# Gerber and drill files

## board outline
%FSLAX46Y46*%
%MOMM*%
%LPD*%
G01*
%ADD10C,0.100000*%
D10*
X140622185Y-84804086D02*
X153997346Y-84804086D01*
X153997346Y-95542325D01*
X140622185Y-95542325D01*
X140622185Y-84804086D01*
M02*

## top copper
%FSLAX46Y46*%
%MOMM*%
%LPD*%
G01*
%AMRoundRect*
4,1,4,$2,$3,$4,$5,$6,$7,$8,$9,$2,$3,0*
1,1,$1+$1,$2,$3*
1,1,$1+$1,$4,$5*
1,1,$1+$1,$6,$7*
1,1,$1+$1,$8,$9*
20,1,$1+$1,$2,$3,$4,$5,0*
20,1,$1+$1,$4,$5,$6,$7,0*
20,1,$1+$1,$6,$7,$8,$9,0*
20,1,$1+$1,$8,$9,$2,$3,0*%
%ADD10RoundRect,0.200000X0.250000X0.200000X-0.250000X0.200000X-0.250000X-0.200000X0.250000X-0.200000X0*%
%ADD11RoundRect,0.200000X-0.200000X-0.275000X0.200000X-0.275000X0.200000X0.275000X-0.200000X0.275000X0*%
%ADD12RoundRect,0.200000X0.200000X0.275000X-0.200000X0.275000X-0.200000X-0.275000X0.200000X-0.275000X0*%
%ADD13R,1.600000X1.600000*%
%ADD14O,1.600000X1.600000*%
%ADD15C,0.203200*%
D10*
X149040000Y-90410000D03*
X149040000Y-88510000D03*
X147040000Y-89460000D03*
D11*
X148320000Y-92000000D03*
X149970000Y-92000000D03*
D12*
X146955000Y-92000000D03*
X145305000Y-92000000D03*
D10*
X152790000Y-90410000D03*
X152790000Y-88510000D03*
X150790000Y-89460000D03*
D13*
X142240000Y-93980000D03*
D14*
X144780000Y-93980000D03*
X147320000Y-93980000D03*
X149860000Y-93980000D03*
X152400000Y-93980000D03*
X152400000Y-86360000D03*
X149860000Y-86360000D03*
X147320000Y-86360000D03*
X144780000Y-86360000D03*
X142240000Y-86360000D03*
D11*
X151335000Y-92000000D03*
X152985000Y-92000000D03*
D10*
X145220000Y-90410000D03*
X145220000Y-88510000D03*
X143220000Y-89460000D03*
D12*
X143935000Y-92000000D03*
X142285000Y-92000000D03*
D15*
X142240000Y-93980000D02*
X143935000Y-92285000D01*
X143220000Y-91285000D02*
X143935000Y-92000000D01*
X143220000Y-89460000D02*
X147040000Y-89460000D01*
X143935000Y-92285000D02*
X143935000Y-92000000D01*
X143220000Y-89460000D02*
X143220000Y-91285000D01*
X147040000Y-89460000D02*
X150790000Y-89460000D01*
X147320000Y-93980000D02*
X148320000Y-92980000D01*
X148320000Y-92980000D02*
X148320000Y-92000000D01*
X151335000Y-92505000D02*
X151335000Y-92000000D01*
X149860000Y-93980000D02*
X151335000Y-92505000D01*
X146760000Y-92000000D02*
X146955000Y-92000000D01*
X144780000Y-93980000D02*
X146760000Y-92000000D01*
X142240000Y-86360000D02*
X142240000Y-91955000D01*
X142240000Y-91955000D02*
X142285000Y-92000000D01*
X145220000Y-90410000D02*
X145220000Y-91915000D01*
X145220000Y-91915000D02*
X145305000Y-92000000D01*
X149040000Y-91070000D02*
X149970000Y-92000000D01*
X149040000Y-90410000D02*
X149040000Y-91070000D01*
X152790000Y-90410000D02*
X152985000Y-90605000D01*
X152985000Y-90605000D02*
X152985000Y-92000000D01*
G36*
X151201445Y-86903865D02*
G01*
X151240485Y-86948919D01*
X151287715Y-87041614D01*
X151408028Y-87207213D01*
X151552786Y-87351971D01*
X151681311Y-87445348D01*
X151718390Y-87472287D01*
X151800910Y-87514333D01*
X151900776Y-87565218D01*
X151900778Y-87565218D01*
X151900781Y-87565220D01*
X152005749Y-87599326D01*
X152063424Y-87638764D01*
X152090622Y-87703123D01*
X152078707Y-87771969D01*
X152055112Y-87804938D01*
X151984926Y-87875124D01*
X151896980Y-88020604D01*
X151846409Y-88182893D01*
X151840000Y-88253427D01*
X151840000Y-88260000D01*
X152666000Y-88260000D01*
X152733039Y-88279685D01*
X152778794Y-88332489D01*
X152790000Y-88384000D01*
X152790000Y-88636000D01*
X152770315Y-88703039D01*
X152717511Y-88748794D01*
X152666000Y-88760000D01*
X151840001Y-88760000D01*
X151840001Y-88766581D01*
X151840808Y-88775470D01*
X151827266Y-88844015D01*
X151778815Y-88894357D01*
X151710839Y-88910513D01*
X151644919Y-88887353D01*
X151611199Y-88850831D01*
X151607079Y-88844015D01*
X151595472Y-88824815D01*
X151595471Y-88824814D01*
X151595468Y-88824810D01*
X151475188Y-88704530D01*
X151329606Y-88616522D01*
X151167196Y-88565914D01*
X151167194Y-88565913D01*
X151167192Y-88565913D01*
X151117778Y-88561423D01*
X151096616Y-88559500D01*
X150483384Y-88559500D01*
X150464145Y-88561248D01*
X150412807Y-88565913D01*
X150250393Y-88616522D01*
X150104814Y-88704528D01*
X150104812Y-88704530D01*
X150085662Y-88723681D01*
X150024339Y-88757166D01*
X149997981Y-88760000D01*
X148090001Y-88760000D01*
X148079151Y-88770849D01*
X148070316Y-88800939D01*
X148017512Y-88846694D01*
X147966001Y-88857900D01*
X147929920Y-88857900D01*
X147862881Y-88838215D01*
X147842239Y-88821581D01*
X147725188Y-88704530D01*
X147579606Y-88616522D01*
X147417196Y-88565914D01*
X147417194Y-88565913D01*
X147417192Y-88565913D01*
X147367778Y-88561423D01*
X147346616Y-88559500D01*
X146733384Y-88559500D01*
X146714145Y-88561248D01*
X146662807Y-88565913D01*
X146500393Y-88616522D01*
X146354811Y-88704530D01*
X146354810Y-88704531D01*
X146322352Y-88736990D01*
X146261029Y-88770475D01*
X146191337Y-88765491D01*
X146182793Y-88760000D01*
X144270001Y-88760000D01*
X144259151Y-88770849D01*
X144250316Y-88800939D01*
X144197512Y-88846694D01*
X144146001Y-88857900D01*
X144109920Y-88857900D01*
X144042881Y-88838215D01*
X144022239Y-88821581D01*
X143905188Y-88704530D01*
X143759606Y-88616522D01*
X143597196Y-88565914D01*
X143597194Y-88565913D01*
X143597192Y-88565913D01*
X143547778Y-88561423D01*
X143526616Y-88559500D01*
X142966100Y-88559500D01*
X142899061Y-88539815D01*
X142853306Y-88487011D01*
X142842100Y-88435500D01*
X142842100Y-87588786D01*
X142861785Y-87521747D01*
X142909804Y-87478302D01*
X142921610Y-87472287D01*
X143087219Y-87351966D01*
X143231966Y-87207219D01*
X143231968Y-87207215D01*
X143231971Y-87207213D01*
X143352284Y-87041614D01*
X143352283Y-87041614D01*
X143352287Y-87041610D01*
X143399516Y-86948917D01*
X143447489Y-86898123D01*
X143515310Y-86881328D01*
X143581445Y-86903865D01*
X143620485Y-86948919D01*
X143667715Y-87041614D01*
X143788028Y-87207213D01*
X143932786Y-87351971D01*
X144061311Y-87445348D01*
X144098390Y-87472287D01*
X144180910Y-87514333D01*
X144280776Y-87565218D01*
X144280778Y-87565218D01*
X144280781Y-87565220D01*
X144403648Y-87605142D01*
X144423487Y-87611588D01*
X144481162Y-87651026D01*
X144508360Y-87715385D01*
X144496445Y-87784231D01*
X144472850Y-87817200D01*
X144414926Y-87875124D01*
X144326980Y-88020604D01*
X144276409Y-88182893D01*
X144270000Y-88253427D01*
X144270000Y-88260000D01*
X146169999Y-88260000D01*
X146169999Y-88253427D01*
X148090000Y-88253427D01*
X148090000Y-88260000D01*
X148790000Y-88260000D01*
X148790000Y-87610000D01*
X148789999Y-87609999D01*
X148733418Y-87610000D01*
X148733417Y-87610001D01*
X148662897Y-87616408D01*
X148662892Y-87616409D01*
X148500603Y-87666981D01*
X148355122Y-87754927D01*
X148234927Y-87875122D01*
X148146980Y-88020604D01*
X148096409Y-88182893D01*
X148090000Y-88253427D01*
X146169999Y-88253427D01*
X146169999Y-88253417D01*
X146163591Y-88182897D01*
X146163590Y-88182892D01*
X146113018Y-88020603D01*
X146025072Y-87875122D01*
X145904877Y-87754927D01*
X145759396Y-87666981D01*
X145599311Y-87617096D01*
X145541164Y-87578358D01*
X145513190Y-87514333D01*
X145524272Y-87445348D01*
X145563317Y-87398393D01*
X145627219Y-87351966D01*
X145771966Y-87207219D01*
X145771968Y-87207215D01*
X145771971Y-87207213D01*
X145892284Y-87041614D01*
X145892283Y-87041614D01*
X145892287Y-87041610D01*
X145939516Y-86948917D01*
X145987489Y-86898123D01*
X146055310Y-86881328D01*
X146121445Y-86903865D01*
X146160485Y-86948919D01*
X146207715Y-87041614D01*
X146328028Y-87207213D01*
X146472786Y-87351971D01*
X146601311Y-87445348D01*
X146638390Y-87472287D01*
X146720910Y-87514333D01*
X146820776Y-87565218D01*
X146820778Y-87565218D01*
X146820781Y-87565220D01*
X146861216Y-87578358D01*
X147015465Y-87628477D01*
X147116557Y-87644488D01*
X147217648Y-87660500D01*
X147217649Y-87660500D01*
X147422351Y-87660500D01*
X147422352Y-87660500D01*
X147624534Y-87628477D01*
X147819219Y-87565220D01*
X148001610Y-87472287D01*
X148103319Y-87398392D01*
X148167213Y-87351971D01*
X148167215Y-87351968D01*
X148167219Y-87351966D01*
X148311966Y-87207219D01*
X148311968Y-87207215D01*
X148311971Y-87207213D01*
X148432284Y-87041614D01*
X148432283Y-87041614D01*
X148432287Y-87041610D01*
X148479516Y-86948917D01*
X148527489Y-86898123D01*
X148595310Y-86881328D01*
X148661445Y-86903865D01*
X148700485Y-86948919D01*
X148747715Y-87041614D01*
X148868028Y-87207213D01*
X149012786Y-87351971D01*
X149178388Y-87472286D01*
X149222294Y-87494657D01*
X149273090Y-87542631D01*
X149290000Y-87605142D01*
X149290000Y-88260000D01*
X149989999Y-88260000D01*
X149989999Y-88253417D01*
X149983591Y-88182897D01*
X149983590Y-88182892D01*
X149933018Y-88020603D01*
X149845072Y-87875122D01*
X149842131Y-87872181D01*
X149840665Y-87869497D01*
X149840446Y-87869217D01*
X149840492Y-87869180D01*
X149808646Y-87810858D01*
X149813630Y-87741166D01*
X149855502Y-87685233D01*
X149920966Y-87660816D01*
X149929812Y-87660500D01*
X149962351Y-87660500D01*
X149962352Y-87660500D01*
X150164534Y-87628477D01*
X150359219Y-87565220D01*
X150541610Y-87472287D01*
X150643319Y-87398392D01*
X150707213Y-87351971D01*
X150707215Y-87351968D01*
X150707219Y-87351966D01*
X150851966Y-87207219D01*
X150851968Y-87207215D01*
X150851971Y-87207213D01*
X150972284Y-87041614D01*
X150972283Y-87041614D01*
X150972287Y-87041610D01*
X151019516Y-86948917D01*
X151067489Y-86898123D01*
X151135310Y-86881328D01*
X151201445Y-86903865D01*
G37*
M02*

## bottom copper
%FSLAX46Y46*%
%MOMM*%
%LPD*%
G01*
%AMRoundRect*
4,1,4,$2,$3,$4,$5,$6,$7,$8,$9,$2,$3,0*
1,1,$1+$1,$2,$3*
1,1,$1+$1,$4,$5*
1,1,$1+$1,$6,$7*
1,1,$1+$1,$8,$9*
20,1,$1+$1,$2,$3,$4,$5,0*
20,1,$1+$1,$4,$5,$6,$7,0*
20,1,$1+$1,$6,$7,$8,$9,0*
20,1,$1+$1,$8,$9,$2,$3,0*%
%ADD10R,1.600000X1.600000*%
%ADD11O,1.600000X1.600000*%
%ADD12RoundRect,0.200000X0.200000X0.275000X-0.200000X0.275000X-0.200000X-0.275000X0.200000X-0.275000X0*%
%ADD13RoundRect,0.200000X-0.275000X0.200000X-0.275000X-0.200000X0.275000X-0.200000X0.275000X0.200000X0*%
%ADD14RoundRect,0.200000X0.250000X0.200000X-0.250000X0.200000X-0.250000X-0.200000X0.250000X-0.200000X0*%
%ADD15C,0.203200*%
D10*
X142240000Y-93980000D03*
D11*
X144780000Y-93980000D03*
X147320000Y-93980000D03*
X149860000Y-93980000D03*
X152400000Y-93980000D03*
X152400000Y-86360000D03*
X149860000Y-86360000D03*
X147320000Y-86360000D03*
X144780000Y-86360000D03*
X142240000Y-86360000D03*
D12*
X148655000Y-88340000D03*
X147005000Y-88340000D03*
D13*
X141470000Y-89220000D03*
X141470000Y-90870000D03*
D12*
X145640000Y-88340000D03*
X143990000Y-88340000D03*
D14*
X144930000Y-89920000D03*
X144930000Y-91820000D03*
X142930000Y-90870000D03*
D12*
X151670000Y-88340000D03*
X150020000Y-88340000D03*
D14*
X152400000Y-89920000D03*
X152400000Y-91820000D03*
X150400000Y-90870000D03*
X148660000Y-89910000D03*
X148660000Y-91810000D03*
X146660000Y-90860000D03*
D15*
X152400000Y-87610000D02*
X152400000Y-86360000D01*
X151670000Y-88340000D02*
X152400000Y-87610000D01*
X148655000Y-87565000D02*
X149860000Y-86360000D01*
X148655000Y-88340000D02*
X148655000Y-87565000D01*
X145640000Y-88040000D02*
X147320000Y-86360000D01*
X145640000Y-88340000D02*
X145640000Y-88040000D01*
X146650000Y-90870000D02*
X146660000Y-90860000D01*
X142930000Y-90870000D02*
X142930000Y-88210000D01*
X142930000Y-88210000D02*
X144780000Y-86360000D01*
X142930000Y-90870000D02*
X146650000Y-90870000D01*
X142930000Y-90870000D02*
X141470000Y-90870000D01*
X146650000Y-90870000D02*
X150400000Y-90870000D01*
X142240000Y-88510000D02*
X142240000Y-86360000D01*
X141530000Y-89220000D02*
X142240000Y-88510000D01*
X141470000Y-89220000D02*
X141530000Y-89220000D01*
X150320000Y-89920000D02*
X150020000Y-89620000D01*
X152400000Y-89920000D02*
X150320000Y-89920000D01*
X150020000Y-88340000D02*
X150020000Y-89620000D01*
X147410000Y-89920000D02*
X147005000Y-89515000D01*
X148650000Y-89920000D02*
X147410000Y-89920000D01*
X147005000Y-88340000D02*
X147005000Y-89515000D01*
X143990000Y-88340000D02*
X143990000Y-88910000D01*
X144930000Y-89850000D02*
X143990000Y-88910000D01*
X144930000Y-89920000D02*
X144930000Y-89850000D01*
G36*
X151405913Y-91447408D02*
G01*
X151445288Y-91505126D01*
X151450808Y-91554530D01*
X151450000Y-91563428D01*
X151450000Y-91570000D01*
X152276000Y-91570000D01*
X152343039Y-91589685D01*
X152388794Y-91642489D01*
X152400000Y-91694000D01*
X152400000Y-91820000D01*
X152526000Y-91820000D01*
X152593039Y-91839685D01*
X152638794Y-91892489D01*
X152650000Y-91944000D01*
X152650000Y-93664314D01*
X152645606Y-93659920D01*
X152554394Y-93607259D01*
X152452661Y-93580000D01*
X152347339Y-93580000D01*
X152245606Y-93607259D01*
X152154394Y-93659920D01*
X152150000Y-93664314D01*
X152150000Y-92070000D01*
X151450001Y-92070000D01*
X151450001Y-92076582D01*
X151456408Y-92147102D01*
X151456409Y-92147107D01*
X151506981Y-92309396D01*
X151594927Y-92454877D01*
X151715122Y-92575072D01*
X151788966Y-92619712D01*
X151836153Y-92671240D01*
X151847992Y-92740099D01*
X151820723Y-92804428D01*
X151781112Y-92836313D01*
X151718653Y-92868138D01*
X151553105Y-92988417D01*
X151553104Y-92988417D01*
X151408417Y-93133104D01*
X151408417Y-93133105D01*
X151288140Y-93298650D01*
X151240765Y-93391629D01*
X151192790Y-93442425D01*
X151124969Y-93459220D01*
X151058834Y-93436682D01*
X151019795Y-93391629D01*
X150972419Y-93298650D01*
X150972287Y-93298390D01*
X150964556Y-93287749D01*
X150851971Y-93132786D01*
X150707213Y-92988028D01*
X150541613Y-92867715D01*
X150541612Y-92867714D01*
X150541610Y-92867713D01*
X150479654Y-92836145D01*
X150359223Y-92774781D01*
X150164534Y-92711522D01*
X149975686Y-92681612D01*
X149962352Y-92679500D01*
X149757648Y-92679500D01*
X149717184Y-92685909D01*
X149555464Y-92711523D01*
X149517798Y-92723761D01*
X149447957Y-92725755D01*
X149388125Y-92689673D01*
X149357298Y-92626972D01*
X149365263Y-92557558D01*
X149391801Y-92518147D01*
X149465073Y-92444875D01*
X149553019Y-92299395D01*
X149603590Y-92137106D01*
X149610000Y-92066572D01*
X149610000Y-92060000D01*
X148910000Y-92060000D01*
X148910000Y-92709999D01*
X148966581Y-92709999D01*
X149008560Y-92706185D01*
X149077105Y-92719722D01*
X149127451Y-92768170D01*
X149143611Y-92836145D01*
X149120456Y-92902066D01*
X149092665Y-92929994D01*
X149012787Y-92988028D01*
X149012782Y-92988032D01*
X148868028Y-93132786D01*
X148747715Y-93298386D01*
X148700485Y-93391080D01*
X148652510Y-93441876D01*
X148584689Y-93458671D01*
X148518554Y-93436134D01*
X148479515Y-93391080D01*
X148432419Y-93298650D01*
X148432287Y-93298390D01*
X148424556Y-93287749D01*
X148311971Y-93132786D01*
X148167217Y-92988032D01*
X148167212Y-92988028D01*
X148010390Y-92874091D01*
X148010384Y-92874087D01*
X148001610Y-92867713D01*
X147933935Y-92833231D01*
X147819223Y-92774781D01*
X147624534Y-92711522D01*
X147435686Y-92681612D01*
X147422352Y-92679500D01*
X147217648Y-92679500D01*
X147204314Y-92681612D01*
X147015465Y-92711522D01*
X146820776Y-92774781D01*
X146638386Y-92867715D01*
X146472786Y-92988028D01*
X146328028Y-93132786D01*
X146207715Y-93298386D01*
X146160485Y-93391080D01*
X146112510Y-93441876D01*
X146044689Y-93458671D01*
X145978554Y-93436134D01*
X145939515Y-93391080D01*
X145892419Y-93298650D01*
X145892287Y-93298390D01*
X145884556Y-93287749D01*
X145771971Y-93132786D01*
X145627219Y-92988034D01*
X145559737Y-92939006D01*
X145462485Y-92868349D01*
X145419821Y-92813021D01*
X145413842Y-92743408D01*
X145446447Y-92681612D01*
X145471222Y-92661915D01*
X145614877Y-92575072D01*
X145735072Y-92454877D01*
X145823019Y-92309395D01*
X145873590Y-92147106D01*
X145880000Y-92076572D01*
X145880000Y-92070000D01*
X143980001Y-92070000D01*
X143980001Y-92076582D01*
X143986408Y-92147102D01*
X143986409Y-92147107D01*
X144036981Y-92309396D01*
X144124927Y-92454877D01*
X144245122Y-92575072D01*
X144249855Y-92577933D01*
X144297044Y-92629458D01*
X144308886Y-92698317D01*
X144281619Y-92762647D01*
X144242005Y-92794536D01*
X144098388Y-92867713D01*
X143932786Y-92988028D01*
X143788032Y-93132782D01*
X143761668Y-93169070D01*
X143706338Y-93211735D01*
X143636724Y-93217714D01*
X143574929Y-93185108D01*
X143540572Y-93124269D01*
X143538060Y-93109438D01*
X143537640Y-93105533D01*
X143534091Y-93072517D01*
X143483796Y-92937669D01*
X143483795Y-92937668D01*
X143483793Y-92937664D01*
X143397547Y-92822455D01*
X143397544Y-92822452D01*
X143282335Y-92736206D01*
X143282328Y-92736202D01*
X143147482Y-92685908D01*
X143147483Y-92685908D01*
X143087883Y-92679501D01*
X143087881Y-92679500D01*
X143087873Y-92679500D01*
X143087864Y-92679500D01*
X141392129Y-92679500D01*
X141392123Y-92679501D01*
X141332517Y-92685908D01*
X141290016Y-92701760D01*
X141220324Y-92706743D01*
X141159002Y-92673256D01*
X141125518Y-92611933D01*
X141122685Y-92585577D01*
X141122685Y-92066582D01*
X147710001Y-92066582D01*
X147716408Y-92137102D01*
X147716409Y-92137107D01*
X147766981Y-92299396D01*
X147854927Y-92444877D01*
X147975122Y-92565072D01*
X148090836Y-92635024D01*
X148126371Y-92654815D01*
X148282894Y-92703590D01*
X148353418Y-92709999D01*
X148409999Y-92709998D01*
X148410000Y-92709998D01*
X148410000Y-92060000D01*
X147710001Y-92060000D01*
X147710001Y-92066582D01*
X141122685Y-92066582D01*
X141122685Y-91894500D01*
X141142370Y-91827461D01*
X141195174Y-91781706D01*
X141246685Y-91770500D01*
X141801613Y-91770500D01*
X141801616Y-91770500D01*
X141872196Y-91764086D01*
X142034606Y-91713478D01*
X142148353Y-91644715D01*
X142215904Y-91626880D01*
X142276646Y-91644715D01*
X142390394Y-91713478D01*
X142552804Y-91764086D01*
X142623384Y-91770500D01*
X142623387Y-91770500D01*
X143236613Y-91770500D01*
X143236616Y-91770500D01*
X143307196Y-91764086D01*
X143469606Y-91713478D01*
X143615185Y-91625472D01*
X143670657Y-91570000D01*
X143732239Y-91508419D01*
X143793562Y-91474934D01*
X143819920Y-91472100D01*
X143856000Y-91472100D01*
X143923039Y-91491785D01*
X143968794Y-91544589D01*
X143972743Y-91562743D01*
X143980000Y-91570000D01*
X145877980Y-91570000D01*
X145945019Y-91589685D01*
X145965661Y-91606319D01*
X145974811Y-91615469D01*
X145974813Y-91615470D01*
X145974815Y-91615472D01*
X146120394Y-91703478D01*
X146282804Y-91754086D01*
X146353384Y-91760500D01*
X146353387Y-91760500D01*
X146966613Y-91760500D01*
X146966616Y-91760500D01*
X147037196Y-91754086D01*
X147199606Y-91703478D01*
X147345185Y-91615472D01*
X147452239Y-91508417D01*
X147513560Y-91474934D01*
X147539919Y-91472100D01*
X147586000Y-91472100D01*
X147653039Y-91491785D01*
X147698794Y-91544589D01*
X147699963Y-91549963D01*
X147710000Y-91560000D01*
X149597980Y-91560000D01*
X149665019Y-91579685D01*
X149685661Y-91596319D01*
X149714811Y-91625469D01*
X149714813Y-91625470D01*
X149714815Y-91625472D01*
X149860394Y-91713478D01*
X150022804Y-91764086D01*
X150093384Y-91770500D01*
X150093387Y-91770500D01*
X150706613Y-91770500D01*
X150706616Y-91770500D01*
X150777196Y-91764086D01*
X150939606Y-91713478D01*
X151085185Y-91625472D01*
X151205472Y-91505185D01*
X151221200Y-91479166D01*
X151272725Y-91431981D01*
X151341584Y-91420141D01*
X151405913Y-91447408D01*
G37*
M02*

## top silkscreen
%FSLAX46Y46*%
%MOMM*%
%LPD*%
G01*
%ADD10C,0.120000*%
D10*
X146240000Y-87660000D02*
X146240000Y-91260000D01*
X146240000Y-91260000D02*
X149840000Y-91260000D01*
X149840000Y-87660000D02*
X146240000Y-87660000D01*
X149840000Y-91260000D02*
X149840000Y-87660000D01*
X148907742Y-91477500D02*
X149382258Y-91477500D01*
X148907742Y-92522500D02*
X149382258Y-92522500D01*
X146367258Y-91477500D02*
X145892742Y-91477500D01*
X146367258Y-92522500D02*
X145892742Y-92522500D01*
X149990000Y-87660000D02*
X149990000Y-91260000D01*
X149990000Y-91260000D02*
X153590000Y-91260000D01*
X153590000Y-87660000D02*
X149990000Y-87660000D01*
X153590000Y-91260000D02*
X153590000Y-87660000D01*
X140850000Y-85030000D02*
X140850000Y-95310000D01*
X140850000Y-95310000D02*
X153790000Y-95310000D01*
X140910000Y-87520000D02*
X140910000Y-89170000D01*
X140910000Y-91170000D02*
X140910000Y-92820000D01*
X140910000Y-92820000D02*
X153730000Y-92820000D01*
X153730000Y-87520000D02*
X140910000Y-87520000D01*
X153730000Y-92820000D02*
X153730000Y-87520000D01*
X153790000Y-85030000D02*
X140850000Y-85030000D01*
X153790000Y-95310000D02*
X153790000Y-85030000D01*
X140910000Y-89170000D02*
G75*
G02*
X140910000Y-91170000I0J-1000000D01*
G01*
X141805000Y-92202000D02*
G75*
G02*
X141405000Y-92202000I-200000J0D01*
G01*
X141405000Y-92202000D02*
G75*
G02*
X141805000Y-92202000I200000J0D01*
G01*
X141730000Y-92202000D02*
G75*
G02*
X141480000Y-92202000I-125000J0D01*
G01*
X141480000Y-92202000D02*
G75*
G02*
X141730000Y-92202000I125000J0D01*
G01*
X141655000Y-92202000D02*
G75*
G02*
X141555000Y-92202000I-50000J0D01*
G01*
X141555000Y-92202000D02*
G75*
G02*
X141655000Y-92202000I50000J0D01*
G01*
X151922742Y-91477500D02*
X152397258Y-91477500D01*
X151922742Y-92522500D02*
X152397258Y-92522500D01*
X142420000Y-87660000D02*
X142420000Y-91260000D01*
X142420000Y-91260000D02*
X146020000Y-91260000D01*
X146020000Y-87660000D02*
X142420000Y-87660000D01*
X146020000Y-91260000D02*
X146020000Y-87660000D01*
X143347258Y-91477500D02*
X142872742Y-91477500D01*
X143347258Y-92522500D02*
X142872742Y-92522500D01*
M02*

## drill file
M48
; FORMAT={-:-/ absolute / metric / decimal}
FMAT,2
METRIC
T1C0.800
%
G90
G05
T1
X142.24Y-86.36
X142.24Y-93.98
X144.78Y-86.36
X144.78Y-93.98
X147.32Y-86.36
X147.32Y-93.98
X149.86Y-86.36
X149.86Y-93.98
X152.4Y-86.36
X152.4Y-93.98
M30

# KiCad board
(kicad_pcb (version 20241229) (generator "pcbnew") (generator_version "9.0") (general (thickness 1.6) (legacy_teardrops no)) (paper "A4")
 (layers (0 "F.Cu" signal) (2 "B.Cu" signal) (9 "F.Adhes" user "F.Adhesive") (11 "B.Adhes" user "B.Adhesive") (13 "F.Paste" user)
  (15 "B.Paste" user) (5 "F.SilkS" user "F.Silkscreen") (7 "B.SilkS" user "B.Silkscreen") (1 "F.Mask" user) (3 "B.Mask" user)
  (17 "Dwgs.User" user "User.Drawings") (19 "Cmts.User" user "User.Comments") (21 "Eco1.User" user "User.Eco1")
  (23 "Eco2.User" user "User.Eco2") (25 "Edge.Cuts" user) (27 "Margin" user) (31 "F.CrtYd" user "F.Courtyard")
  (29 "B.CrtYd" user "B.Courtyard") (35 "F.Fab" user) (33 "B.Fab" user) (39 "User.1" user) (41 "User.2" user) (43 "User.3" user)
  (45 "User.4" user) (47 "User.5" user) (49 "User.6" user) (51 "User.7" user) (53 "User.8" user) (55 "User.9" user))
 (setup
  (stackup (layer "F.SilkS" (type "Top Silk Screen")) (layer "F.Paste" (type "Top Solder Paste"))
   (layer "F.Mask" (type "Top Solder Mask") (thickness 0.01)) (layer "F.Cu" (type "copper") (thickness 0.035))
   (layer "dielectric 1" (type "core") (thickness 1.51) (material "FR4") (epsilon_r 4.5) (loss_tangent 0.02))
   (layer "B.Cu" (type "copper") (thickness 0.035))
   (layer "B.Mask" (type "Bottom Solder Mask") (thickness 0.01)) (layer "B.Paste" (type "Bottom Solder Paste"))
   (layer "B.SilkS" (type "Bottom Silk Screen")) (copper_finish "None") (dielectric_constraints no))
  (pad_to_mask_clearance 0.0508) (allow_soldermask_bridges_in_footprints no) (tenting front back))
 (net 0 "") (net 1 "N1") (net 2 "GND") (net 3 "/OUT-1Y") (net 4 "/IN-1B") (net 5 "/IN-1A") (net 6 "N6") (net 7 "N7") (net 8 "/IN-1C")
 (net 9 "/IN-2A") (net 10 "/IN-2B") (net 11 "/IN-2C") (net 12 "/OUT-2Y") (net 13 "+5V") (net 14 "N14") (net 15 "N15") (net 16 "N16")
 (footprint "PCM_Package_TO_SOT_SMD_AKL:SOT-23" (layer "F.Cu") (at 148.04 89.46 180)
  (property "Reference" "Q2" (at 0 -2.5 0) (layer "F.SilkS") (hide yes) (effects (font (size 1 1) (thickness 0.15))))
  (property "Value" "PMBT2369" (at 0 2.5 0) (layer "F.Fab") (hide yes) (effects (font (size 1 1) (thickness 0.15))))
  (fp_line (start 1.8 1.8) (end 1.8 -1.8) (stroke (width 0.12) (type solid)) (layer "F.SilkS"))
  (fp_line (start 1.8 -1.8) (end -1.8 -1.8) (stroke (width 0.12) (type solid)) (layer "F.SilkS"))
  (fp_line (start -1.8 1.8) (end 1.8 1.8) (stroke (width 0.12) (type solid)) (layer "F.SilkS"))
  (fp_line (start -1.8 -1.8) (end -1.8 1.8) (stroke (width 0.12) (type solid)) (layer "F.SilkS"))
  (pad "1" smd roundrect (at -1 -0.95 180) (size 0.9 0.8) (layers "F.Cu" "F.Mask" "F.Paste") (roundrect_rratio 0.25) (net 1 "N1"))
  (pad "2" smd roundrect (at -1 0.95 180) (size 0.9 0.8) (layers "F.Cu" "F.Mask" "F.Paste") (roundrect_rratio 0.25) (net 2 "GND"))
  (pad "3" smd roundrect (at 1 0 180) (size 0.9 0.8) (layers "F.Cu" "F.Mask" "F.Paste") (roundrect_rratio 0.25) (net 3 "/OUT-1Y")))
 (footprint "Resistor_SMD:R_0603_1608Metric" (layer "F.Cu") (at 149.145 92)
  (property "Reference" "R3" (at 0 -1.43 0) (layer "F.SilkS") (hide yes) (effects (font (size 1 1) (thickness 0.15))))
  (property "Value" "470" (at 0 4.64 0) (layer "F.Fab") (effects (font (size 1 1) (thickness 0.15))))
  (fp_line (start -0.237258 -0.5225) (end 0.237258 -0.5225) (stroke (width 0.12) (type solid)) (layer "F.SilkS"))
  (fp_line (start -0.237258 0.5225) (end 0.237258 0.5225) (stroke (width 0.12) (type solid)) (layer "F.SilkS"))
  (pad "1" smd roundrect (at -0.825 0) (size 0.8 0.95) (layers "F.Cu" "F.Mask" "F.Paste") (roundrect_rratio 0.25) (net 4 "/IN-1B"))
  (pad "2" smd roundrect (at 0.825 0) (size 0.8 0.95) (layers "F.Cu" "F.Mask" "F.Paste") (roundrect_rratio 0.25) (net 1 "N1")))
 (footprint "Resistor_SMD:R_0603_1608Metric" (layer "F.Cu") (at 146.13 92 180)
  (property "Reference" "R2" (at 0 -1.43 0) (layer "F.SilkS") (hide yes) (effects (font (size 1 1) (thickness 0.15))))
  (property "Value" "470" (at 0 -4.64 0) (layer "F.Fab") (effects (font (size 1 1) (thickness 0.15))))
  (fp_line (start -0.237258 0.5225) (end 0.237258 0.5225) (stroke (width 0.12) (type solid)) (layer "F.SilkS"))
  (fp_line (start -0.237258 -0.5225) (end 0.237258 -0.5225) (stroke (width 0.12) (type solid)) (layer "F.SilkS"))
  (pad "1" smd roundrect (at -0.825 0 180) (size 0.8 0.95) (layers "F.Cu" "F.Mask" "F.Paste") (roundrect_rratio 0.25) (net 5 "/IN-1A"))
  (pad "2" smd roundrect (at 0.825 0 180) (size 0.8 0.95) (layers "F.Cu" "F.Mask" "F.Paste") (roundrect_rratio 0.25) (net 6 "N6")))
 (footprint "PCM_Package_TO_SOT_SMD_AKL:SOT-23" (layer "F.Cu") (at 151.79 89.46 180)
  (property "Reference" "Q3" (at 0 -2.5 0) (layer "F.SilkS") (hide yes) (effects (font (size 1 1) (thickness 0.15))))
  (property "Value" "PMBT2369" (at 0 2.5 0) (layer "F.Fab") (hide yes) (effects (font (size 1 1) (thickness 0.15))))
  (fp_line (start 1.8 1.8) (end 1.8 -1.8) (stroke (width 0.12) (type solid)) (layer "F.SilkS"))
  (fp_line (start 1.8 -1.8) (end -1.8 -1.8) (stroke (width 0.12) (type solid)) (layer "F.SilkS"))
  (fp_line (start -1.8 1.8) (end 1.8 1.8) (stroke (width 0.12) (type solid)) (layer "F.SilkS"))
  (fp_line (start -1.8 -1.8) (end -1.8 1.8) (stroke (width 0.12) (type solid)) (layer "F.SilkS"))
  (pad "1" smd roundrect (at -1 -0.95 180) (size 0.9 0.8) (layers "F.Cu" "F.Mask" "F.Paste") (roundrect_rratio 0.25) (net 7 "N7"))
  (pad "2" smd roundrect (at -1 0.95 180) (size 0.9 0.8) (layers "F.Cu" "F.Mask" "F.Paste") (roundrect_rratio 0.25) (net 2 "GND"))
  (pad "3" smd roundrect (at 1 0 180) (size 0.9 0.8) (layers "F.Cu" "F.Mask" "F.Paste") (roundrect_rratio 0.25) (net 3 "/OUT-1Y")))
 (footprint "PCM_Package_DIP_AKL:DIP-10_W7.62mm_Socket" (layer "F.Cu") (at 142.24 93.98 90)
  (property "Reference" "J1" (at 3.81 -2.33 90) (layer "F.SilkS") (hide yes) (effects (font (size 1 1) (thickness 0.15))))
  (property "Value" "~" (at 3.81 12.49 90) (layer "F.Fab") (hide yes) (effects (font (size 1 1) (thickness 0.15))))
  (fp_line (start 8.95 -1.39) (end -1.33 -1.39) (stroke (width 0.12) (type solid)) (layer "F.SilkS"))
  (fp_line (start -1.33 -1.39) (end -1.33 11.55) (stroke (width 0.12) (type solid)) (layer "F.SilkS"))
  (fp_line (start 6.46 -1.33) (end 4.81 -1.33) (stroke (width 0.12) (type solid)) (layer "F.SilkS"))
  (fp_line (start 2.81 -1.33) (end 1.16 -1.33) (stroke (width 0.12) (type solid)) (layer "F.SilkS"))
  (fp_line (start 1.16 -1.33) (end 1.16 11.49) (stroke (width 0.12) (type solid)) (layer "F.SilkS"))
  (fp_line (start 6.46 11.49) (end 6.46 -1.33) (stroke (width 0.12) (type solid)) (layer "F.SilkS"))
  (fp_line (start 1.16 11.49) (end 6.46 11.49) (stroke (width 0.12) (type solid)) (layer "F.SilkS"))
  (fp_line (start 8.95 11.55) (end 8.95 -1.39) (stroke (width 0.12) (type solid)) (layer "F.SilkS"))
  (fp_line (start -1.33 11.55) (end 8.95 11.55) (stroke (width 0.12) (type solid)) (layer "F.SilkS"))
  (fp_arc (start 4.81 -1.33) (mid 3.81 -0.33) (end 2.81 -1.33) (stroke (width 0.12) (type solid)) (layer "F.SilkS"))
  (fp_circle (center 1.778 -0.635) (end 1.978 -0.635) (stroke (width 0.12) (type solid)) (fill no) (layer "F.SilkS"))
  (fp_circle (center 1.778 -0.635) (end 1.903 -0.635) (stroke (width 0.12) (type solid)) (fill no) (layer "F.SilkS"))
  (fp_circle (center 1.778 -0.635) (end 1.828 -0.635) (stroke (width 0.12) (type solid)) (fill no) (layer "F.SilkS"))
  (pad "1" thru_hole rect (at 0 0 90) (size 1.6 1.6) (drill 0.8) (layers "*.Cu" "*.Mask") (remove_unused_layers no) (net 3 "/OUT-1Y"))
  (pad "2" thru_hole oval (at 0 2.54 90) (size 1.6 1.6) (drill 0.8) (layers "*.Cu" "*.Mask") (remove_unused_layers no) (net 5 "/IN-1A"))
  (pad "3" thru_hole oval (at 0 5.08 90) (size 1.6 1.6) (drill 0.8) (layers "*.Cu" "*.Mask") (remove_unused_layers no) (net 4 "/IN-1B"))
  (pad "4" thru_hole oval (at 0 7.62 90) (size 1.6 1.6) (drill 0.8) (layers "*.Cu" "*.Mask") (remove_unused_layers no) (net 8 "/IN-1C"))
  (pad "5" thru_hole oval (at 0 10.16 90) (size 1.6 1.6) (drill 0.8) (layers "*.Cu" "*.Mask") (remove_unused_layers no) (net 2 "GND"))
  (pad "6" thru_hole oval (at 7.62 10.16 90) (size 1.6 1.6) (drill 0.8) (layers "*.Cu" "*.Mask") (remove_unused_layers no) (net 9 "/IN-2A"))
  (pad "7" thru_hole oval (at 7.62 7.62 90) (size 1.6 1.6) (drill 0.8) (layers "*.Cu" "*.Mask") (remove_unused_layers no) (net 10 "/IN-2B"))
  (pad "8" thru_hole oval (at 7.62 5.08 90) (size 1.6 1.6) (drill 0.8) (layers "*.Cu" "*.Mask") (remove_unused_layers no) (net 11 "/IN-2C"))
  (pad "9" thru_hole oval (at 7.62 2.54 90) (size 1.6 1.6) (drill 0.8) (layers "*.Cu" "*.Mask") (remove_unused_layers no) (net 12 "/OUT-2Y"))
  (pad "10" thru_hole oval (at 7.62 0 90) (size 1.6 1.6) (drill 0.8) (layers "*.Cu" "*.Mask") (remove_unused_layers no) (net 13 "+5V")))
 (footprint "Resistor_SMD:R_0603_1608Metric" (layer "F.Cu") (at 152.16 92)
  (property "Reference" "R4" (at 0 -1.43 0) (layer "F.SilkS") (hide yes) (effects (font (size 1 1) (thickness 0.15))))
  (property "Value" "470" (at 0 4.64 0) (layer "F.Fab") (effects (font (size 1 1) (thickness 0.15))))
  (fp_line (start -0.237258 -0.5225) (end 0.237258 -0.5225) (stroke (width 0.12) (type solid)) (layer "F.SilkS"))
  (fp_line (start -0.237258 0.5225) (end 0.237258 0.5225) (stroke (width 0.12) (type solid)) (layer "F.SilkS"))
  (pad "1" smd roundrect (at -0.825 0) (size 0.8 0.95) (layers "F.Cu" "F.Mask" "F.Paste") (roundrect_rratio 0.25) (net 8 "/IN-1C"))
  (pad "2" smd roundrect (at 0.825 0) (size 0.8 0.95) (layers "F.Cu" "F.Mask" "F.Paste") (roundrect_rratio 0.25) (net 7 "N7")))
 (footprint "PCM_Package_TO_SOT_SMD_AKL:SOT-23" (layer "F.Cu") (at 144.22 89.46 180)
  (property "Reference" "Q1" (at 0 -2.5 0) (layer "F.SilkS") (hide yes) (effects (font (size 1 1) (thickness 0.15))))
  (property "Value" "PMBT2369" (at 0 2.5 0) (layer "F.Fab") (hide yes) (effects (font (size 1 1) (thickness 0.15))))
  (fp_line (start 1.8 1.8) (end 1.8 -1.8) (stroke (width 0.12) (type solid)) (layer "F.SilkS"))
  (fp_line (start 1.8 -1.8) (end -1.8 -1.8) (stroke (width 0.12) (type solid)) (layer "F.SilkS"))
  (fp_line (start -1.8 1.8) (end 1.8 1.8) (stroke (width 0.12) (type solid)) (layer "F.SilkS"))
  (fp_line (start -1.8 -1.8) (end -1.8 1.8) (stroke (width 0.12) (type solid)) (layer "F.SilkS"))
  (pad "1" smd roundrect (at -1 -0.95 180) (size 0.9 0.8) (layers "F.Cu" "F.Mask" "F.Paste") (roundrect_rratio 0.25) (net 6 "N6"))
  (pad "2" smd roundrect (at -1 0.95 180) (size 0.9 0.8) (layers "F.Cu" "F.Mask" "F.Paste") (roundrect_rratio 0.25) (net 2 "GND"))
  (pad "3" smd roundrect (at 1 0 180) (size 0.9 0.8) (layers "F.Cu" "F.Mask" "F.Paste") (roundrect_rratio 0.25) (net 3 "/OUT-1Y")))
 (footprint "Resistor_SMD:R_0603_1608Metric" (layer "F.Cu") (at 143.11 92 180)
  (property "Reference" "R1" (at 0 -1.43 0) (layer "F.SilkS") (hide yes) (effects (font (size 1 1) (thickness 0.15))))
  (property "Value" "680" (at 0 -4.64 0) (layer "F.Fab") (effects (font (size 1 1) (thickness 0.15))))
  (fp_line (start -0.237258 0.5225) (end 0.237258 0.5225) (stroke (width 0.12) (type solid)) (layer "F.SilkS"))
  (fp_line (start -0.237258 -0.5225) (end 0.237258 -0.5225) (stroke (width 0.12) (type solid)) (layer "F.SilkS"))
  (pad "1" smd roundrect (at -0.825 0 180) (size 0.8 0.95) (layers "F.Cu" "F.Mask" "F.Paste") (roundrect_rratio 0.25) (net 3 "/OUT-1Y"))
  (pad "2" smd roundrect (at 0.825 0 180) (size 0.8 0.95) (layers "F.Cu" "F.Mask" "F.Paste") (roundrect_rratio 0.25) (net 13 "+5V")))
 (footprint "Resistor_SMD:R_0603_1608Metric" (layer "B.Cu") (at 147.83 88.34 180)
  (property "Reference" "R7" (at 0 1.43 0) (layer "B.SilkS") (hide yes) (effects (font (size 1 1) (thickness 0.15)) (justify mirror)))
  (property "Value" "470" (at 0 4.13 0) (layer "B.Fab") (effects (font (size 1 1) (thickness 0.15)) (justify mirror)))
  (pad "1" smd roundrect (at -0.825 0 180) (size 0.8 0.95) (layers "B.Cu" "B.Mask" "B.Paste") (roundrect_rratio 0.25) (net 10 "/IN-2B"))
  (pad "2" smd roundrect (at 0.825 0 180) (size 0.8 0.95) (layers "B.Cu" "B.Mask" "B.Paste") (roundrect_rratio 0.25) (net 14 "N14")))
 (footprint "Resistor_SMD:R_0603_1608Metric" (layer "B.Cu") (at 141.47 90.045 -90)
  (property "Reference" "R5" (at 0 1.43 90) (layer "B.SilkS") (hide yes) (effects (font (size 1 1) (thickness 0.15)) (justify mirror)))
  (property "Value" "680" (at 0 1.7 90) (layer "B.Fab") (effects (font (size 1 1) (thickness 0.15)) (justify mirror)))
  (pad "1" smd roundrect (at -0.825 0 270) (size 0.8 0.95) (layers "B.Cu" "B.Mask" "B.Paste") (roundrect_rratio 0.25) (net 13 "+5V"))
  (pad "2" smd roundrect (at 0.825 0 270) (size 0.8 0.95) (layers "B.Cu" "B.Mask" "B.Paste") (roundrect_rratio 0.25) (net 12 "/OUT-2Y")))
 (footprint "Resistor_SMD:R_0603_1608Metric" (layer "B.Cu") (at 144.815 88.34 180)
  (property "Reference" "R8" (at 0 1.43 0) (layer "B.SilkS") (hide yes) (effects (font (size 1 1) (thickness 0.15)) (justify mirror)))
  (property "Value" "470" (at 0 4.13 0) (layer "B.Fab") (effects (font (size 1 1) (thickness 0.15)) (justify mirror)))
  (pad "1" smd roundrect (at -0.825 0 180) (size 0.8 0.95) (layers "B.Cu" "B.Mask" "B.Paste") (roundrect_rratio 0.25) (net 11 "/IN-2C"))
  (pad "2" smd roundrect (at 0.825 0 180) (size 0.8 0.95) (layers "B.Cu" "B.Mask" "B.Paste") (roundrect_rratio 0.25) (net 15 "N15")))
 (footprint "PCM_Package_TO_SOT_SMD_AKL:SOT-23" (layer "B.Cu") (at 143.93 90.87 180)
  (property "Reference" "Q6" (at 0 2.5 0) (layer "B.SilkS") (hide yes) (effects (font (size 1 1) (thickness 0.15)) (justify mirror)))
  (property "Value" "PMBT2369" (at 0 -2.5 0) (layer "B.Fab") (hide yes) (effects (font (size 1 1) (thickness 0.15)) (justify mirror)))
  (pad "1" smd roundrect (at -1 0.95 180) (size 0.9 0.8) (layers "B.Cu" "B.Mask" "B.Paste") (roundrect_rratio 0.25) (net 15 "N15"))
  (pad "2" smd roundrect (at -1 -0.95 180) (size 0.9 0.8) (layers "B.Cu" "B.Mask" "B.Paste") (roundrect_rratio 0.25) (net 2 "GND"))
  (pad "3" smd roundrect (at 1 0 180) (size 0.9 0.8) (layers "B.Cu" "B.Mask" "B.Paste") (roundrect_rratio 0.25) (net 12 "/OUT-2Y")))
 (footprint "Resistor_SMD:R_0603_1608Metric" (layer "B.Cu") (at 150.845 88.34 180)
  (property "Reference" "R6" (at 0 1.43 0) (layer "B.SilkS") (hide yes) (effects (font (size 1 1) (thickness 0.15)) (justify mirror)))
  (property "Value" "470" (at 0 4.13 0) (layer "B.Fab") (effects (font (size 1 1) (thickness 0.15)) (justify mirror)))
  (pad "1" smd roundrect (at -0.825 0 180) (size 0.8 0.95) (layers "B.Cu" "B.Mask" "B.Paste") (roundrect_rratio 0.25) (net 9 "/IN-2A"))
  (pad "2" smd roundrect (at 0.825 0 180) (size 0.8 0.95) (layers "B.Cu" "B.Mask" "B.Paste") (roundrect_rratio 0.25) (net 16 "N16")))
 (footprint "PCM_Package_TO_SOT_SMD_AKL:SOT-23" (layer "B.Cu") (at 151.4 90.87 180)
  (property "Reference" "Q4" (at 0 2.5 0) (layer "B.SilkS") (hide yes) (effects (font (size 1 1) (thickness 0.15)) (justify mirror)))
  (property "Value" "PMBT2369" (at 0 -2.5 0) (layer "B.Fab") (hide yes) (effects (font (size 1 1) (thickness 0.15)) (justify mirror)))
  (pad "1" smd roundrect (at -1 0.95 180) (size 0.9 0.8) (layers "B.Cu" "B.Mask" "B.Paste") (roundrect_rratio 0.25) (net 16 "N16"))
  (pad "2" smd roundrect (at -1 -0.95 180) (size 0.9 0.8) (layers "B.Cu" "B.Mask" "B.Paste") (roundrect_rratio 0.25) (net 2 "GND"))
  (pad "3" smd roundrect (at 1 0 180) (size 0.9 0.8) (layers "B.Cu" "B.Mask" "B.Paste") (roundrect_rratio 0.25) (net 12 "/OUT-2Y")))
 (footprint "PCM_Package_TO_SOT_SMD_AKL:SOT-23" (layer "B.Cu") (at 147.66 90.86 180)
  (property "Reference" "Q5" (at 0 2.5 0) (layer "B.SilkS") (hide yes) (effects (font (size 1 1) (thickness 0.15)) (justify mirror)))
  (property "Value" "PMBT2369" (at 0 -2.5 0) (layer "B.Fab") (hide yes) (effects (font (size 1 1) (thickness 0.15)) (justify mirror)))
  (pad "1" smd roundrect (at -1 0.95 180) (size 0.9 0.8) (layers "B.Cu" "B.Mask" "B.Paste") (roundrect_rratio 0.25) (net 14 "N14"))
  (pad "2" smd roundrect (at -1 -0.95 180) (size 0.9 0.8) (layers "B.Cu" "B.Mask" "B.Paste") (roundrect_rratio 0.25) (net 2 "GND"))
  (pad "3" smd roundrect (at 1 0 180) (size 0.9 0.8) (layers "B.Cu" "B.Mask" "B.Paste") (roundrect_rratio 0.25) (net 12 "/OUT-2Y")))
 (gr_rect (start 140.622185 84.804086) (end 153.997346 95.542325) (stroke (width 0.1) (type default)) (fill no) (layer "Edge.Cuts"))
 (segment (start 142.24 93.98) (end 143.935 92.285) (width 0.2032) (layer "F.Cu") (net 3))
 (segment (start 143.22 91.285) (end 143.935 92) (width 0.2032) (layer "F.Cu") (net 3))
 (segment (start 143.22 89.46) (end 147.04 89.46) (width 0.2032) (layer "F.Cu") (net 3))
 (segment (start 143.935 92.285) (end 143.935 92) (width 0.2032) (layer "F.Cu") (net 3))
 (segment (start 143.22 89.46) (end 143.22 91.285) (width 0.2032) (layer "F.Cu") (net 3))
 (segment (start 147.04 89.46) (end 150.79 89.46) (width 0.2032) (layer "F.Cu") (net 3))
 (segment (start 147.32 93.98) (end 148.32 92.98) (width 0.2032) (layer "F.Cu") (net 4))
 (segment (start 148.32 92.98) (end 148.32 92) (width 0.2032) (layer "F.Cu") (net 4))
 (segment (start 151.335 92.505) (end 151.335 92) (width 0.2032) (layer "F.Cu") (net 8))
 (segment (start 149.86 93.98) (end 151.335 92.505) (width 0.2032) (layer "F.Cu") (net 8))
 (segment (start 146.76 92) (end 146.955 92) (width 0.2032) (layer "F.Cu") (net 5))
 (segment (start 144.78 93.98) (end 146.76 92) (width 0.2032) (layer "F.Cu") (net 5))
 (segment (start 152.4 87.61) (end 152.4 86.36) (width 0.2032) (layer "B.Cu") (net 9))
 (segment (start 151.67 88.34) (end 152.4 87.61) (width 0.2032) (layer "B.Cu") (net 9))
 (segment (start 148.655 87.565) (end 149.86 86.36) (width 0.2032) (layer "B.Cu") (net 10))
 (segment (start 148.655 88.34) (end 148.655 87.565) (width 0.2032) (layer "B.Cu") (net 10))
 (segment (start 145.64 88.04) (end 147.32 86.36) (width 0.2032) (layer "B.Cu") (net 11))
 (segment (start 145.64 88.34) (end 145.64 88.04) (width 0.2032) (layer "B.Cu") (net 11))
 (segment (start 146.65 90.87) (end 146.66 90.86) (width 0.2032) (layer "B.Cu") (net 12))
 (segment (start 142.93 90.87) (end 142.93 88.21) (width 0.2032) (layer "B.Cu") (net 12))
 (segment (start 142.93 88.21) (end 144.78 86.36) (width 0.2032) (layer "B.Cu") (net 12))
 (segment (start 142.93 90.87) (end 146.65 90.87) (width 0.2032) (layer "B.Cu") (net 12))
 (segment (start 142.93 90.87) (end 141.47 90.87) (width 0.2032) (layer "B.Cu") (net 12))
 (segment (start 146.65 90.87) (end 150.4 90.87) (width 0.2032) (layer "B.Cu") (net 12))
 (segment (start 142.24 86.36) (end 142.24 91.955) (width 0.2032) (layer "F.Cu") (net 13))
 (segment (start 142.24 91.955) (end 142.285 92) (width 0.2032) (layer "F.Cu") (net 13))
 (segment (start 142.24 88.51) (end 142.24 86.36) (width 0.2032) (layer "B.Cu") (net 13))
 (segment (start 141.53 89.22) (end 142.24 88.51) (width 0.2032) (layer "B.Cu") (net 13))
 (segment (start 141.47 89.22) (end 141.53 89.22) (width 0.2032) (layer "B.Cu") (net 13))
 (segment (start 145.22 90.41) (end 145.22 91.915) (width 0.2032) (layer "F.Cu") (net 6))
 (segment (start 145.22 91.915) (end 145.305 92) (width 0.2032) (layer "F.Cu") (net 6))
 (segment (start 149.04 91.07) (end 149.97 92) (width 0.2032) (layer "F.Cu") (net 1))
 (segment (start 149.04 90.41) (end 149.04 91.07) (width 0.2032) (layer "F.Cu") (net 1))
 (segment (start 152.79 90.41) (end 152.985 90.605) (width 0.2032) (layer "F.Cu") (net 7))
 (segment (start 152.985 90.605) (end 152.985 92) (width 0.2032) (layer "F.Cu") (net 7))
 (segment (start 150.32 89.92) (end 150.02 89.62) (width 0.2032) (layer "B.Cu") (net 16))
 (segment (start 152.4 89.92) (end 150.32 89.92) (width 0.2032) (layer "B.Cu") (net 16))
 (segment (start 150.02 88.34) (end 150.02 89.62) (width 0.2032) (layer "B.Cu") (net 16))
 (segment (start 147.41 89.92) (end 147.005 89.515) (width 0.2032) (layer "B.Cu") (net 14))
 (segment (start 148.65 89.92) (end 147.41 89.92) (width 0.2032) (layer "B.Cu") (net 14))
 (segment (start 147.005 88.34) (end 147.005 89.515) (width 0.2032) (layer "B.Cu") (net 14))
 (segment (start 143.99 88.34) (end 143.99 88.91) (width 0.2032) (layer "B.Cu") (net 15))
 (segment (start 144.93 89.85) (end 143.99 88.91) (width 0.2032) (layer "B.Cu") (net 15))
 (segment (start 144.93 89.92) (end 144.93 89.85) (width 0.2032) (layer "B.Cu") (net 15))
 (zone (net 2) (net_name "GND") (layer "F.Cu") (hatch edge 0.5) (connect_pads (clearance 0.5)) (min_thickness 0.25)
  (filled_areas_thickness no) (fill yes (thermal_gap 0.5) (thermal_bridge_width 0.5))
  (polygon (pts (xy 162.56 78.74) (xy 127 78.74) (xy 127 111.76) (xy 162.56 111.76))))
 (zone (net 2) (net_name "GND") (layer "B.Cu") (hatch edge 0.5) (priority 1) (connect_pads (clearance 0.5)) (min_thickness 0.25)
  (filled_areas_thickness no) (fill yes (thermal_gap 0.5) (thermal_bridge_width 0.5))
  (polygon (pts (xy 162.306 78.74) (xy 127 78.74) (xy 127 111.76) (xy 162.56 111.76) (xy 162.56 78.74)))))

